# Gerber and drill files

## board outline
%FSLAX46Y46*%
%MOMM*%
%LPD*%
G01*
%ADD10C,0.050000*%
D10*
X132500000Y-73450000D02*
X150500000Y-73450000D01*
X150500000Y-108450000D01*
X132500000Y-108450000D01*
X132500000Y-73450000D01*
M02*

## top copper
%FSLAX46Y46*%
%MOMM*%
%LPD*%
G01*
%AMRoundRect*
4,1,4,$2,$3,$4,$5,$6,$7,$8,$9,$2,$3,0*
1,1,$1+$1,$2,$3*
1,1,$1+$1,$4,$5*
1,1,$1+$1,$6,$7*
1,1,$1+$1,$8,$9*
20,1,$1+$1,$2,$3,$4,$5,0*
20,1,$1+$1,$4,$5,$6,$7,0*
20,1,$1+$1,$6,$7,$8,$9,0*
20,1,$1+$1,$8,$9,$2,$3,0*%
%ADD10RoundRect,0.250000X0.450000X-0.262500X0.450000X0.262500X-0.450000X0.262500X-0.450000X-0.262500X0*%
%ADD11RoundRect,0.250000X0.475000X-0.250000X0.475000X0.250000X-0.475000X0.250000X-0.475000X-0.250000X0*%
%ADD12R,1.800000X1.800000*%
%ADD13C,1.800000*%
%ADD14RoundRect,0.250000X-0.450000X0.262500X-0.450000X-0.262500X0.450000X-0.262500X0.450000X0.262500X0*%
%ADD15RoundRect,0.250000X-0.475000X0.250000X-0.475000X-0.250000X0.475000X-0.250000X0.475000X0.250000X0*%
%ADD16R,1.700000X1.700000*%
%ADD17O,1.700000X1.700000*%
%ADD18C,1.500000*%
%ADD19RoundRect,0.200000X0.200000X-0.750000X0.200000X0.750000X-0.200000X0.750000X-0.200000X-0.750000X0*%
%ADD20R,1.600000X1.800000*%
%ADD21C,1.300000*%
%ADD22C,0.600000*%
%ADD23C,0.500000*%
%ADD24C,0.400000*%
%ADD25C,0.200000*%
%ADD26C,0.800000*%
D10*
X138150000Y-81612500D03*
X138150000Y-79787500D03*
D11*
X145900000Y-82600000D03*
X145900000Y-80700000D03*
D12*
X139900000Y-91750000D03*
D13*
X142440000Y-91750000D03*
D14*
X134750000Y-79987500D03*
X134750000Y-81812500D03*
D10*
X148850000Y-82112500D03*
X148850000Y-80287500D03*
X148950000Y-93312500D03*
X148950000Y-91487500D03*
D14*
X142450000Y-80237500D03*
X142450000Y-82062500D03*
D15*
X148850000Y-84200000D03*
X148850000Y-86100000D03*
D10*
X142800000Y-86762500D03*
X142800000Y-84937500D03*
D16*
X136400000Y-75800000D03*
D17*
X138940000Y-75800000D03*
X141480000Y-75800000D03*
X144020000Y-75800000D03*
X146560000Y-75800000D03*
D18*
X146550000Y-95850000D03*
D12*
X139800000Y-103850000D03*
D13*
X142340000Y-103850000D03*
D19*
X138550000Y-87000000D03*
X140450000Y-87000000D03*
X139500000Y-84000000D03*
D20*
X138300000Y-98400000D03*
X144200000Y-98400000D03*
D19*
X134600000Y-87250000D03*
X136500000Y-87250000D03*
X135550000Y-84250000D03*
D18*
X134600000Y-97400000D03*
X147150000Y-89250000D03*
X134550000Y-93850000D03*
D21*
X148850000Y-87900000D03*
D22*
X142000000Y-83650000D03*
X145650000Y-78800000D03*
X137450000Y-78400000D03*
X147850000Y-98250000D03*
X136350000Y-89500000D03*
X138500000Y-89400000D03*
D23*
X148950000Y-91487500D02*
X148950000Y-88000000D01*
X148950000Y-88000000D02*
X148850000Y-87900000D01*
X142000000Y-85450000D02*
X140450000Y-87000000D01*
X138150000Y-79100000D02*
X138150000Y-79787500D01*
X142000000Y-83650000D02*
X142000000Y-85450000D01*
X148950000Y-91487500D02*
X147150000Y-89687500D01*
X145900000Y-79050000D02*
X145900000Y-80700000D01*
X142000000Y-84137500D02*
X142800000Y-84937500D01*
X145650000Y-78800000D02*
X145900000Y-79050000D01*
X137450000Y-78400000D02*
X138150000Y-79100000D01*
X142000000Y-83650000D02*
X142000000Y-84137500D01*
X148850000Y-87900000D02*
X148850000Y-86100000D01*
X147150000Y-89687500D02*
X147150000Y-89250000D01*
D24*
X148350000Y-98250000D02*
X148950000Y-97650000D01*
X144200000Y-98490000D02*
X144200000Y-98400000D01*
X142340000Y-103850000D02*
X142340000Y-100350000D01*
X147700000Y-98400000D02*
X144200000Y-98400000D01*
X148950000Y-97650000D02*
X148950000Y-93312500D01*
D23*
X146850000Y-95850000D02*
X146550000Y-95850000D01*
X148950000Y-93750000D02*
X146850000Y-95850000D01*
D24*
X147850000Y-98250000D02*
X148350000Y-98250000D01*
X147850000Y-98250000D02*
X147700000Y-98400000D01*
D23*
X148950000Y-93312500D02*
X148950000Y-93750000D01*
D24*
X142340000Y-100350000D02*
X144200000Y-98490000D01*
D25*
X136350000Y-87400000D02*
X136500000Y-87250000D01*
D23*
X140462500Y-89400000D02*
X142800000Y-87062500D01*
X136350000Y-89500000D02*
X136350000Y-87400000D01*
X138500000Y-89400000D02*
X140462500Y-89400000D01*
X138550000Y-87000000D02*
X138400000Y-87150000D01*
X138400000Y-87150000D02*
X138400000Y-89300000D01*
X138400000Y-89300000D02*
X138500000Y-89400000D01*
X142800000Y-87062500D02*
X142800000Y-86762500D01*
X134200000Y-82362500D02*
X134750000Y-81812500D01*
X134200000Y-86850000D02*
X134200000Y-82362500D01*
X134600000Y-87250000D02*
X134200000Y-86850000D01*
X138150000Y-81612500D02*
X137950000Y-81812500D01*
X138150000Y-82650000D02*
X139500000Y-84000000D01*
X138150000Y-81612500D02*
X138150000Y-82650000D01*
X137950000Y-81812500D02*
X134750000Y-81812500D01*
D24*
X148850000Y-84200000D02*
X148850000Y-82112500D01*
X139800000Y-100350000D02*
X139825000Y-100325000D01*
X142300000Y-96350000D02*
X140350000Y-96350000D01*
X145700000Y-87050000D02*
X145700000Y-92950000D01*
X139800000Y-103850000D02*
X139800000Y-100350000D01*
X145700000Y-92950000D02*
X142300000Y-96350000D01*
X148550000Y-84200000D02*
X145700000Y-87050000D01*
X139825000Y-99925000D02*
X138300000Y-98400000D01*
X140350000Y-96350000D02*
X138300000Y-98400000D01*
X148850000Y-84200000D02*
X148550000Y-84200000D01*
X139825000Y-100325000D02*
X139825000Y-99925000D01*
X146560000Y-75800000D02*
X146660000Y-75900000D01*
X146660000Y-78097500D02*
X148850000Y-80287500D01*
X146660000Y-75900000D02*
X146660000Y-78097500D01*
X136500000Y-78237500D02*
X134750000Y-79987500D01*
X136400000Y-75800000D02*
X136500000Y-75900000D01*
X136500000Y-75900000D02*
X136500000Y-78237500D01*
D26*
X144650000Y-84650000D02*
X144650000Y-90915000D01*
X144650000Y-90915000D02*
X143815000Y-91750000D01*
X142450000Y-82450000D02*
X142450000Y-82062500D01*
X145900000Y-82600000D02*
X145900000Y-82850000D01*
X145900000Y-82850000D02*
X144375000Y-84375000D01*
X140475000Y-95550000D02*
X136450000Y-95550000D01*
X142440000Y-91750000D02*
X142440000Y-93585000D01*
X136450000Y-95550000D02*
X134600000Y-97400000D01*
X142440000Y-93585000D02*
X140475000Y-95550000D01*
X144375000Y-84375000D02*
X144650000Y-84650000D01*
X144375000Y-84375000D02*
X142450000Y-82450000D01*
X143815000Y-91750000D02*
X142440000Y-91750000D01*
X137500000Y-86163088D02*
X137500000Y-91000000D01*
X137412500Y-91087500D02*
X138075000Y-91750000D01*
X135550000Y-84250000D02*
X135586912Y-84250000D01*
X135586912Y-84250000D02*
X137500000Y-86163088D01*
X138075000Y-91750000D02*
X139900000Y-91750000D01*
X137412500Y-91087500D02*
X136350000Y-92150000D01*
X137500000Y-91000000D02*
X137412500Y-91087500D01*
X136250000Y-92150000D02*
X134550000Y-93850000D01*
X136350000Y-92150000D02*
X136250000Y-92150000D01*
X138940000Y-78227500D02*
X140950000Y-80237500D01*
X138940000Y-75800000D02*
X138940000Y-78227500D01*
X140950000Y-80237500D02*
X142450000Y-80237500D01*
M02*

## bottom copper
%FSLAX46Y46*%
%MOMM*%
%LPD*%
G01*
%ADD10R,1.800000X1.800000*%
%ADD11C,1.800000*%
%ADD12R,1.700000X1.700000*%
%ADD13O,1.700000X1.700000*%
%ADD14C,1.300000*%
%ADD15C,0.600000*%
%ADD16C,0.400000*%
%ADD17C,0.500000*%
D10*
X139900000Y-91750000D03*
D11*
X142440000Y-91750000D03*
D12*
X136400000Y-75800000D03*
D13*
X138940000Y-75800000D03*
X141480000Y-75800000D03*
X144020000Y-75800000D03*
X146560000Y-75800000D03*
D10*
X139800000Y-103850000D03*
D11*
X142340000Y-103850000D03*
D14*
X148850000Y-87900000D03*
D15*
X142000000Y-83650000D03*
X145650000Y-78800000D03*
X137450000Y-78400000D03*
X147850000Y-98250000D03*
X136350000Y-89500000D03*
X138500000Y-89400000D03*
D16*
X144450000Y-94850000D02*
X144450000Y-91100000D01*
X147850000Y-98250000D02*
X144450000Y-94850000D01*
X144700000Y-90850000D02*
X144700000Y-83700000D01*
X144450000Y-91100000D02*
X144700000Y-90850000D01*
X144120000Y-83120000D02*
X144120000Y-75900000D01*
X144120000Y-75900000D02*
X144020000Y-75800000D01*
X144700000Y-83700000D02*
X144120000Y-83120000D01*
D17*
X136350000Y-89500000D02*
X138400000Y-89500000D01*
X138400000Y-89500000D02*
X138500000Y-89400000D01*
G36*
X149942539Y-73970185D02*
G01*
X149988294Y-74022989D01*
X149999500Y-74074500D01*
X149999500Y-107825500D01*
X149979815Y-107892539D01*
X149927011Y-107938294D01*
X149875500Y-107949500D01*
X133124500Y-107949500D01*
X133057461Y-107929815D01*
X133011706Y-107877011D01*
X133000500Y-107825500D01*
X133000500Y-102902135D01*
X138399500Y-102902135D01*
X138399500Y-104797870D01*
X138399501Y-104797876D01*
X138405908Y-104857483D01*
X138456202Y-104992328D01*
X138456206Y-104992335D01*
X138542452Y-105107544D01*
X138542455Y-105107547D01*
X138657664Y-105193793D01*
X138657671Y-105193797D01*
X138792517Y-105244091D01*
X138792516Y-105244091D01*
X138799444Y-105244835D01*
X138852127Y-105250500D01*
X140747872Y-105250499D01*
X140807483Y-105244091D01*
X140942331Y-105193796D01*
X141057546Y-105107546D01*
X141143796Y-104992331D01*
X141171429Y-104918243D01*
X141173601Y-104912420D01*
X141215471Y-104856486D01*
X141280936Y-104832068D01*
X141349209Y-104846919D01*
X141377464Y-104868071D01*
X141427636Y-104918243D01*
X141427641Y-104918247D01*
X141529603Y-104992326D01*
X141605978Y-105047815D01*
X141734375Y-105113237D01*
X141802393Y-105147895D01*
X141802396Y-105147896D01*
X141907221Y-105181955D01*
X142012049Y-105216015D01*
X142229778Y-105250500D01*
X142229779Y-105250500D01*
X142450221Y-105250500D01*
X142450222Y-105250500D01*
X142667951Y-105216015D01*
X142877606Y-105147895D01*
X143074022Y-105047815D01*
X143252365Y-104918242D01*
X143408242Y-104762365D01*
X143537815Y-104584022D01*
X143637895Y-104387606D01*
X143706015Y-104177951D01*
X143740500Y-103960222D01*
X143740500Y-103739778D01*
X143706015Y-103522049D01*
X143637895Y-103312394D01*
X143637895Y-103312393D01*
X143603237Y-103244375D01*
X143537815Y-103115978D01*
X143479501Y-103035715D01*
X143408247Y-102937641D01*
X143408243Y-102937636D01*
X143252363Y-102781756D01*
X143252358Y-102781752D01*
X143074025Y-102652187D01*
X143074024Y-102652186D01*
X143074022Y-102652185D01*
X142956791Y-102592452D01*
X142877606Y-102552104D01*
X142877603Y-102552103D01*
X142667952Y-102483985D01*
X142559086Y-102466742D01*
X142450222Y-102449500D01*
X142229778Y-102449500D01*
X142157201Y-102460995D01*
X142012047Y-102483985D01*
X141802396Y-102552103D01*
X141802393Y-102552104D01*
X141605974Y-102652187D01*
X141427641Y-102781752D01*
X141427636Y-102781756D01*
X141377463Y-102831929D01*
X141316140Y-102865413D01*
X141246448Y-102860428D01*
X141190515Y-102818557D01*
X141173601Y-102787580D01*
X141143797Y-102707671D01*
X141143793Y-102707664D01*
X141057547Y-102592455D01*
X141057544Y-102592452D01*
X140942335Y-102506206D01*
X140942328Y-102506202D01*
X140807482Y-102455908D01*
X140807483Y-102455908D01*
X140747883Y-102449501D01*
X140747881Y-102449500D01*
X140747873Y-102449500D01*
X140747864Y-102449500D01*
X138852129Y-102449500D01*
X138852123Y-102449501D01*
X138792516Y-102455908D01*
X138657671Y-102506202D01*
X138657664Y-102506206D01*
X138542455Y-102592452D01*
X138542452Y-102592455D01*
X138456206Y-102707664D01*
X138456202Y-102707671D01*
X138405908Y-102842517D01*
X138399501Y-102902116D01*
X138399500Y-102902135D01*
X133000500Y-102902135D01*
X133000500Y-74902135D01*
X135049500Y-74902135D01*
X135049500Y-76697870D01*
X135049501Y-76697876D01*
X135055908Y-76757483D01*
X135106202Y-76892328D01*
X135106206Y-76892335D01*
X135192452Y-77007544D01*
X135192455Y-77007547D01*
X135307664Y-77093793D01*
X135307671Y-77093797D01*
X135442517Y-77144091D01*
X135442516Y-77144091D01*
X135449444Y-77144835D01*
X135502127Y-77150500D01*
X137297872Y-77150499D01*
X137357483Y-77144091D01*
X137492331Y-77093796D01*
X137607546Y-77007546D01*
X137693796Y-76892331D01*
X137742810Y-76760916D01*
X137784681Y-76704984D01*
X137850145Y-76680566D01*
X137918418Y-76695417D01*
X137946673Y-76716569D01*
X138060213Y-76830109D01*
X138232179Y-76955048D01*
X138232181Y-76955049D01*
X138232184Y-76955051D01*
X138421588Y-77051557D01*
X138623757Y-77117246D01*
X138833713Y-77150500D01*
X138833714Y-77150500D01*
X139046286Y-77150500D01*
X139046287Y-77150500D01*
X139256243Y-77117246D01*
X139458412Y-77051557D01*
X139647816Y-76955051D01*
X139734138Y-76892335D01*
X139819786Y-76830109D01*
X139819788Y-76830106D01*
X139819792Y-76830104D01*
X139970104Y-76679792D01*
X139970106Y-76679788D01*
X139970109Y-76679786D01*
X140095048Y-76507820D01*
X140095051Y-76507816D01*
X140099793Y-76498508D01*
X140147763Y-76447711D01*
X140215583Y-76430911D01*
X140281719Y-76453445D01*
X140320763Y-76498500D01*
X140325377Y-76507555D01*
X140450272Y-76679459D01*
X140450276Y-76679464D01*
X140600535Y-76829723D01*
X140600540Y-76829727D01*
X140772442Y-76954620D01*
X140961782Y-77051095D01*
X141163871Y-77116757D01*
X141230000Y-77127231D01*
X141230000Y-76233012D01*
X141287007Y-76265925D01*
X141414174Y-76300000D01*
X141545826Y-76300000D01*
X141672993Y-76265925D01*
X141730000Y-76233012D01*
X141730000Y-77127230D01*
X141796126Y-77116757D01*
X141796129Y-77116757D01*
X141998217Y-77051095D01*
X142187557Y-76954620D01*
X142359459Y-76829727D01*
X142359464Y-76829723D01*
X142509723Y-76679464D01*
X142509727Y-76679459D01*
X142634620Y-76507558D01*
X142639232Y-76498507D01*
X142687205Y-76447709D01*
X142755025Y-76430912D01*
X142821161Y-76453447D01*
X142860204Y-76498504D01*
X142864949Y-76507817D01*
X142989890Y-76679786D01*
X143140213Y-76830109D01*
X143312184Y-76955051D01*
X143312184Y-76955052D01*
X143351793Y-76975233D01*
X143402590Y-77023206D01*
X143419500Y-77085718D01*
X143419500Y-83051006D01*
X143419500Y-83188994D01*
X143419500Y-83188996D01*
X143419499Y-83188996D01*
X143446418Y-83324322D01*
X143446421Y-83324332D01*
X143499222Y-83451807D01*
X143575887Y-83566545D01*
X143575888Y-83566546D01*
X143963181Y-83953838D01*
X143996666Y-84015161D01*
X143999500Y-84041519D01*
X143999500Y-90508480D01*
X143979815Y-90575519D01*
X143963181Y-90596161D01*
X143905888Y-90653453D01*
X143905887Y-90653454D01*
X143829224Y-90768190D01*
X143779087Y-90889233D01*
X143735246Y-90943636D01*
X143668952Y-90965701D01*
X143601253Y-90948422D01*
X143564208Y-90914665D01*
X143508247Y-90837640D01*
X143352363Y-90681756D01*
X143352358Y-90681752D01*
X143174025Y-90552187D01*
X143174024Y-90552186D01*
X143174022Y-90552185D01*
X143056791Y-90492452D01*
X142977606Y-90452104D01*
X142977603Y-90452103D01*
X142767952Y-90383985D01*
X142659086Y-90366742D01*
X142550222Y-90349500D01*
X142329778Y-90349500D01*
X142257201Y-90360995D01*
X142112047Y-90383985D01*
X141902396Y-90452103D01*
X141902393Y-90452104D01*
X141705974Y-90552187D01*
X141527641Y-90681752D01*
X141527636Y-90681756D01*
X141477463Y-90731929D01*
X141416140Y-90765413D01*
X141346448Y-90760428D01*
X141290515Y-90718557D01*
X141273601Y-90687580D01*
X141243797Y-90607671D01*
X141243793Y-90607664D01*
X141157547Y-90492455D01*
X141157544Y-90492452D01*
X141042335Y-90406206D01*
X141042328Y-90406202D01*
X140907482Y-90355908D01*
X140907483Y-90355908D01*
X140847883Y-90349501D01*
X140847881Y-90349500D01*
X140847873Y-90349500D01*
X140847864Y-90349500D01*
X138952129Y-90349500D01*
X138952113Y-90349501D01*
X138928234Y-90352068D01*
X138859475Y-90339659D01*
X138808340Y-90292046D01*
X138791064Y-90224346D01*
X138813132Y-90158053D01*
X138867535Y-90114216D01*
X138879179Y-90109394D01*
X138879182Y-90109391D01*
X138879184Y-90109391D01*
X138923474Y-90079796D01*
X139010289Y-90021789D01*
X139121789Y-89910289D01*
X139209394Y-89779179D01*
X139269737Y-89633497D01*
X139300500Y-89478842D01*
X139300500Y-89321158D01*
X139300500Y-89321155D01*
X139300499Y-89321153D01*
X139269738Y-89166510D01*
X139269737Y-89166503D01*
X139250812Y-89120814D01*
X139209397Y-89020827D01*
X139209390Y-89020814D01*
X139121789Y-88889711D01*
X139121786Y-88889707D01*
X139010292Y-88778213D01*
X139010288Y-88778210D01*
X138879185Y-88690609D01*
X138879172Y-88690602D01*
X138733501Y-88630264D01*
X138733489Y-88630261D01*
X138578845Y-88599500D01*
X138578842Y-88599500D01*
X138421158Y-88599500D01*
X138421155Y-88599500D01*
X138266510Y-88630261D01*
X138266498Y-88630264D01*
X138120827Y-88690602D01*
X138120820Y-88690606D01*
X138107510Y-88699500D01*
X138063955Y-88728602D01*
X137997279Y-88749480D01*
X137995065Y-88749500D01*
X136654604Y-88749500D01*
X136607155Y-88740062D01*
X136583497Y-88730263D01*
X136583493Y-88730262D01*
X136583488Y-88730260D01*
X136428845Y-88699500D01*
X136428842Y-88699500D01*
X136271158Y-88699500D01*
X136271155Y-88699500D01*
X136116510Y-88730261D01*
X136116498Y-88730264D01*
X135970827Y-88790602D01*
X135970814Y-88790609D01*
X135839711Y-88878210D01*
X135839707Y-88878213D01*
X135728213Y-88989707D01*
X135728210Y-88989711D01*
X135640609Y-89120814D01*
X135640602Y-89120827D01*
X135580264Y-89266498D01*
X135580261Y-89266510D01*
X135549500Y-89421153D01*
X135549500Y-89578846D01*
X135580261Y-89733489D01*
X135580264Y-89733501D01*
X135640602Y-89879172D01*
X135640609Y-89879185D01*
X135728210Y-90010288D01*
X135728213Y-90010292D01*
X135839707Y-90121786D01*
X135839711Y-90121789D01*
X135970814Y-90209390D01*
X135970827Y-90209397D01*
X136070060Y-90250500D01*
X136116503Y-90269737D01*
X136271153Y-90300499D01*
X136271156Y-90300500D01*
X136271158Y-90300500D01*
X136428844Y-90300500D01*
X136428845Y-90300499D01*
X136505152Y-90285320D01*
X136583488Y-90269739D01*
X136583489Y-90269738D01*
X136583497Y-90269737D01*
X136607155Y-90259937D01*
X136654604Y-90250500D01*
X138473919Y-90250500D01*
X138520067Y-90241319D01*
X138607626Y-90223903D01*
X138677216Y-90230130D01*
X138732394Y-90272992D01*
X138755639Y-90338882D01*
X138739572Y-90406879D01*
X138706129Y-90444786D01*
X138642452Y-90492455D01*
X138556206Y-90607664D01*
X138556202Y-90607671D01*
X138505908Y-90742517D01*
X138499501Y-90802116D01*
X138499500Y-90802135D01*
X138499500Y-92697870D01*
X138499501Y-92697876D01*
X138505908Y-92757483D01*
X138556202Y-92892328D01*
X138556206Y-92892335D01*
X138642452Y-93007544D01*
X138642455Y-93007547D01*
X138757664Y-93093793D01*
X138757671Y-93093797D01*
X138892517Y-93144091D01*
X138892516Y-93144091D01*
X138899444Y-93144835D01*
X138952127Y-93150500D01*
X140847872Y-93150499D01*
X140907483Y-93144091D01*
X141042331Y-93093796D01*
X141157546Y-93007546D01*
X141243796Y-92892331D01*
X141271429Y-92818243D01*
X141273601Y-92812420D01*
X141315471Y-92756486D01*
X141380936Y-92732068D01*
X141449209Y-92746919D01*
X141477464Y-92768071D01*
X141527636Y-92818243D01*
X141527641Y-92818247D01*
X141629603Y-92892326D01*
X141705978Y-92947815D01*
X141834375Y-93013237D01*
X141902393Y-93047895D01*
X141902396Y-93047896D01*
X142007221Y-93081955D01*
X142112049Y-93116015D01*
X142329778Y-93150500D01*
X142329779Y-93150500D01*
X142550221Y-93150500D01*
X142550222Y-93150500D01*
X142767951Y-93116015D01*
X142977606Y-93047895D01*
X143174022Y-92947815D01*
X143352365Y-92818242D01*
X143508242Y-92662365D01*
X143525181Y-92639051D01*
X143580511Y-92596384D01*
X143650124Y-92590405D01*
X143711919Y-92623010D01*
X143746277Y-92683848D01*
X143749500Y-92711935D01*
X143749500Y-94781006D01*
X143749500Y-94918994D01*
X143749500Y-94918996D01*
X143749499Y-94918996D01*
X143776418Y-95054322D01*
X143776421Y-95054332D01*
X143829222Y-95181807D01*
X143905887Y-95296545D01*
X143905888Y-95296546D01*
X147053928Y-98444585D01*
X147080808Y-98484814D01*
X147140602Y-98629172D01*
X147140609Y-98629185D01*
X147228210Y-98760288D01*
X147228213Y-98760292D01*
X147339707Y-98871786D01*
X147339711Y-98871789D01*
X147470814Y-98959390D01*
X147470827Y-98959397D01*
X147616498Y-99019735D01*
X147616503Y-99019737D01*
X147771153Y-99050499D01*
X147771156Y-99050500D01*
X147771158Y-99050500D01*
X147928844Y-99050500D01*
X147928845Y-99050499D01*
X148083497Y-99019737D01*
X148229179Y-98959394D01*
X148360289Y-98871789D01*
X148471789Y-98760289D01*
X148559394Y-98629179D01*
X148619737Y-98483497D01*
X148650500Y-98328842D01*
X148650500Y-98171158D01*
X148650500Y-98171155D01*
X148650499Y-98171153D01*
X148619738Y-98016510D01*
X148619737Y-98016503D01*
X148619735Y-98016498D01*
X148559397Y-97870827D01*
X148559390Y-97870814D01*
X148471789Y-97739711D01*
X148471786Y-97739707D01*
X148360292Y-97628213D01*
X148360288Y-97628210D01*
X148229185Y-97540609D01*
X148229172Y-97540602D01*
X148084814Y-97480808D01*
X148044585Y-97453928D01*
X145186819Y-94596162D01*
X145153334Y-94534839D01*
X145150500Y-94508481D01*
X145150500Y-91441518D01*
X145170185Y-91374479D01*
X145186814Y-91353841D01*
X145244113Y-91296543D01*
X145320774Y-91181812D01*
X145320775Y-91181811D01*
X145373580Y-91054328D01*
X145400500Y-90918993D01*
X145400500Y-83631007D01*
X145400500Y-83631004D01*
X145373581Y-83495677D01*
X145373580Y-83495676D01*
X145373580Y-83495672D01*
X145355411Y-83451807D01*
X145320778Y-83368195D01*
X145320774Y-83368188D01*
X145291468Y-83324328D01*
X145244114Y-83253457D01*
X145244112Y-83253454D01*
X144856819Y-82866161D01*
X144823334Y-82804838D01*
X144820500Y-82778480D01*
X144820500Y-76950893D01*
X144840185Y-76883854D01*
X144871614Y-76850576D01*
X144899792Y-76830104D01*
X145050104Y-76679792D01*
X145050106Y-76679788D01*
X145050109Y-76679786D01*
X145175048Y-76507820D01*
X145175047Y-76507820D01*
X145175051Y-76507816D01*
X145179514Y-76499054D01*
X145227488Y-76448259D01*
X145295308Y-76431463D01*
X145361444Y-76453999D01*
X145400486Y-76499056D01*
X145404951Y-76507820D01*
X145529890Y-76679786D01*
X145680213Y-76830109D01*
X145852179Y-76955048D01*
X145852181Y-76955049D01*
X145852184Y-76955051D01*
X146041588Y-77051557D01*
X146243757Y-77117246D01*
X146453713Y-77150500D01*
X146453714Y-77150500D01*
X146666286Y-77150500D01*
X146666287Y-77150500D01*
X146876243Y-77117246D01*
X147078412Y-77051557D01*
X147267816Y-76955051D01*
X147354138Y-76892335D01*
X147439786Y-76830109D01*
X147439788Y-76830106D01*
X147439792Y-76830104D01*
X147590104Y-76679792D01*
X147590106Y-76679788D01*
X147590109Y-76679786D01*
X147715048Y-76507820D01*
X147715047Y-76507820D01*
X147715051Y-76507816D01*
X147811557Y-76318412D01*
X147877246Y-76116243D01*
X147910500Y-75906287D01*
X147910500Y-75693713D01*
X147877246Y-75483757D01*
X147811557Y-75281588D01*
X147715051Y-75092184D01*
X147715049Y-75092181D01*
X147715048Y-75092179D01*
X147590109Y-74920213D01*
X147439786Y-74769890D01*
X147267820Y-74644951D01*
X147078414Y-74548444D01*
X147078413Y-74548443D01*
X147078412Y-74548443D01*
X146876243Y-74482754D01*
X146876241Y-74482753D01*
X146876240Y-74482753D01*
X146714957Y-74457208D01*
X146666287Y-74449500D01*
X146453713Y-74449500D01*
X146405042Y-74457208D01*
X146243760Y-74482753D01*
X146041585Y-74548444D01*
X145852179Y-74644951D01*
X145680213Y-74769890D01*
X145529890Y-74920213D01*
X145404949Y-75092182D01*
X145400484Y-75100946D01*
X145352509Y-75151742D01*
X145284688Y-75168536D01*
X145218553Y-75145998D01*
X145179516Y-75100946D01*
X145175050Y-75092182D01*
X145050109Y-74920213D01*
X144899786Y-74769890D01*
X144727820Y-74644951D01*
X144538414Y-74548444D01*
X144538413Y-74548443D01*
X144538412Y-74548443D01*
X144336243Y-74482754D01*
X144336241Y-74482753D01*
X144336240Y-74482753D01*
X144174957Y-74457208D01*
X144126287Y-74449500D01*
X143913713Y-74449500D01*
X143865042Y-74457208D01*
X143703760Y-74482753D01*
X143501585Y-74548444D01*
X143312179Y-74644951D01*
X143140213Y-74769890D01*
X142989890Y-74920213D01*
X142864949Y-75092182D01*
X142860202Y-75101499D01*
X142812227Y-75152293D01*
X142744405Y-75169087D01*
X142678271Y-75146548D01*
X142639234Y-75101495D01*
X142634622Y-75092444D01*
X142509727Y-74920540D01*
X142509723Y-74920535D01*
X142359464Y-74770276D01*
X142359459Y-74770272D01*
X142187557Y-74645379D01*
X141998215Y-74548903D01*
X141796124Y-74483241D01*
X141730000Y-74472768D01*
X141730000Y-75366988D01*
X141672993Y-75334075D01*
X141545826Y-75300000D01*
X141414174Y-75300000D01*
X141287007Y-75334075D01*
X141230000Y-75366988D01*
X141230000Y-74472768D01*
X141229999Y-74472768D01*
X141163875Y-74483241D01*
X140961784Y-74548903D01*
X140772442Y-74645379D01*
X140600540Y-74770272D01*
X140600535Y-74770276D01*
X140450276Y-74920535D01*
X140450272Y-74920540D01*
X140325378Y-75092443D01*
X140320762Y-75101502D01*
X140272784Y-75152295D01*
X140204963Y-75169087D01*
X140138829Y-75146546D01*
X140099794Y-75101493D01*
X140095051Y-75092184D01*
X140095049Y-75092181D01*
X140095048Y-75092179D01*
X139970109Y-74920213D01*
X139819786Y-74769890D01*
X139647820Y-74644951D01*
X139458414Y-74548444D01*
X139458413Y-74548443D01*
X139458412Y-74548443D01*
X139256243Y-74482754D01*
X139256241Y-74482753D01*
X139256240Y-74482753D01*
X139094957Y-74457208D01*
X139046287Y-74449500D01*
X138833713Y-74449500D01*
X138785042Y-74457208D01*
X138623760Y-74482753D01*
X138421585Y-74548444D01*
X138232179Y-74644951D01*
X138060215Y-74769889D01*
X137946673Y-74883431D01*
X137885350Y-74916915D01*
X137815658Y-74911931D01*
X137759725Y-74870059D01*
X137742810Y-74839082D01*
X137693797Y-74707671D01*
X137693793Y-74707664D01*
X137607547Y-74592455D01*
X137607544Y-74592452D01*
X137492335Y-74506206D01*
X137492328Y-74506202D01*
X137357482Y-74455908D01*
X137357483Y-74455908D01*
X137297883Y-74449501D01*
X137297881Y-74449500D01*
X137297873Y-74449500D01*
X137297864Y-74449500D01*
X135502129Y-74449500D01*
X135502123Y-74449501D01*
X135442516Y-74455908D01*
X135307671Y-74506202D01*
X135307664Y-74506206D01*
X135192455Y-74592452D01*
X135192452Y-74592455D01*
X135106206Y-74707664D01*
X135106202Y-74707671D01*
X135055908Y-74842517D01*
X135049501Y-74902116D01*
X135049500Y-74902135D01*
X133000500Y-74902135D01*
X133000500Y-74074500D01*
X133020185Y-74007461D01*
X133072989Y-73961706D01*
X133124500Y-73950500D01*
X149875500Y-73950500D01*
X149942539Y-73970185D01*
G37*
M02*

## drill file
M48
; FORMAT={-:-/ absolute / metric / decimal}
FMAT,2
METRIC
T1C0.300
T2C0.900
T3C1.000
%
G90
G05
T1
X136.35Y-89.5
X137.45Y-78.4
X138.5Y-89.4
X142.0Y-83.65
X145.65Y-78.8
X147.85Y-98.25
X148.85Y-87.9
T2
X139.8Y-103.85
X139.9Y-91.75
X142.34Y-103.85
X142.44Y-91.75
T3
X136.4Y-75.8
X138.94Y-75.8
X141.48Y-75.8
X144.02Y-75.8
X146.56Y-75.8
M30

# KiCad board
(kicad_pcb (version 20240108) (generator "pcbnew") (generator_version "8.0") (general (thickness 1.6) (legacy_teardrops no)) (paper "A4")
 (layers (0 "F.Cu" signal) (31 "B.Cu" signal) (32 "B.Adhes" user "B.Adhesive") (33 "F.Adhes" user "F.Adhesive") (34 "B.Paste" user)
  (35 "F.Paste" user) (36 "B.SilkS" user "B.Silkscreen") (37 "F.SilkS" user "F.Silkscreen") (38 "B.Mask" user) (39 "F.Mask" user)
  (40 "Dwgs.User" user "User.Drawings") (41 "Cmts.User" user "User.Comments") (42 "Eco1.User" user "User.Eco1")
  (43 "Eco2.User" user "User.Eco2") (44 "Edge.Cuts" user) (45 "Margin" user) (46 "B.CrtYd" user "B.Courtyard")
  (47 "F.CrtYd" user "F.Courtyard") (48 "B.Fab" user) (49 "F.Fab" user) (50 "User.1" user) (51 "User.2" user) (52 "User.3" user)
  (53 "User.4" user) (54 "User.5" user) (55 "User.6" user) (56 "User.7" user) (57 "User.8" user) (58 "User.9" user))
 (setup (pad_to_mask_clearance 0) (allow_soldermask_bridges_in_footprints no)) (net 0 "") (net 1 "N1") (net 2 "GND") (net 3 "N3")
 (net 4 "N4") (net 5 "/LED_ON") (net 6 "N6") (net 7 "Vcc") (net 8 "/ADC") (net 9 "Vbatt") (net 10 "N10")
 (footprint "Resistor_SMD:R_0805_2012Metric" (layer "F.Cu") (at 138.15 80.7 90)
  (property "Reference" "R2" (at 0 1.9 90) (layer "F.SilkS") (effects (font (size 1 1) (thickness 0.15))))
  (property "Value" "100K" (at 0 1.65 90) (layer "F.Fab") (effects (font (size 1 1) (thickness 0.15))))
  (pad "1" smd roundrect (at -0.9125 0 90) (size 1.025 1.4) (layers "F.Cu" "F.Paste" "F.Mask") (roundrect_rratio 0.243902) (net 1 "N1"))
  (pad "2" smd roundrect (at 0.9125 0 90) (size 1.025 1.4) (layers "F.Cu" "F.Paste" "F.Mask") (roundrect_rratio 0.243902) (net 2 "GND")))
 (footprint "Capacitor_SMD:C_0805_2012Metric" (layer "F.Cu") (at 145.9 81.65 90)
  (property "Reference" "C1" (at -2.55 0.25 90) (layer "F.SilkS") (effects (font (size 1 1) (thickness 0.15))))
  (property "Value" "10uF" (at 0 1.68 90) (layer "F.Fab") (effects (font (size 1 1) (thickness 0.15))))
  (pad "1" smd roundrect (at -0.95 0 90) (size 1 1.45) (layers "F.Cu" "F.Paste" "F.Mask") (roundrect_rratio 0.25) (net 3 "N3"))
  (pad "2" smd roundrect (at 0.95 0 90) (size 1 1.45) (layers "F.Cu" "F.Paste" "F.Mask") (roundrect_rratio 0.25) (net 2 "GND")))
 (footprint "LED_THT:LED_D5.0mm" (layer "F.Cu") (at 139.9 91.75)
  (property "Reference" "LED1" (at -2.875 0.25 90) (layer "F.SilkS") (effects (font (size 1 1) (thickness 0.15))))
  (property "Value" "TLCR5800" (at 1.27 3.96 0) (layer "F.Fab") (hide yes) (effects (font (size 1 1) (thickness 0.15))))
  (pad "1" thru_hole rect (at 0 0) (size 1.8 1.8) (drill 0.9) (layers "*.Cu" "*.Mask") (remove_unused_layers no) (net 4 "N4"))
  (pad "2" thru_hole circle (at 2.54 0) (size 1.8 1.8) (drill 0.9) (layers "*.Cu" "*.Mask") (remove_unused_layers no) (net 3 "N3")))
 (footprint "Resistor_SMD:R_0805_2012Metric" (layer "F.Cu") (at 134.75 80.9 -90)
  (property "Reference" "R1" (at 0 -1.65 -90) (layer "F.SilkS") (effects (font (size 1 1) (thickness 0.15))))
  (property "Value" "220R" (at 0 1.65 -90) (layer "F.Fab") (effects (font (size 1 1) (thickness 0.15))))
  (pad "1" smd roundrect (at -0.9125 0 270) (size 1.025 1.4) (layers "F.Cu" "F.Paste" "F.Mask") (roundrect_rratio 0.243902)
   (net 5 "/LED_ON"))
  (pad "2" smd roundrect (at 0.9125 0 270) (size 1.025 1.4) (layers "F.Cu" "F.Paste" "F.Mask") (roundrect_rratio 0.243902) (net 1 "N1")))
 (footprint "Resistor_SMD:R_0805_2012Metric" (layer "F.Cu") (at 148.85 81.2 90)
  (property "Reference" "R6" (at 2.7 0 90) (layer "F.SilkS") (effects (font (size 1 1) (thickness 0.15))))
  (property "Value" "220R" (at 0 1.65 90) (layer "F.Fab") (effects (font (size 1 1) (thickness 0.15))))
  (pad "1" smd roundrect (at -0.9125 0 90) (size 1.025 1.4) (layers "F.Cu" "F.Paste" "F.Mask") (roundrect_rratio 0.243902) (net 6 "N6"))
  (pad "2" smd roundrect (at 0.9125 0 90) (size 1.025 1.4) (layers "F.Cu" "F.Paste" "F.Mask") (roundrect_rratio 0.243902) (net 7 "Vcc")))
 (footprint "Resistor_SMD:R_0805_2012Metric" (layer "F.Cu") (at 148.95 92.4 90)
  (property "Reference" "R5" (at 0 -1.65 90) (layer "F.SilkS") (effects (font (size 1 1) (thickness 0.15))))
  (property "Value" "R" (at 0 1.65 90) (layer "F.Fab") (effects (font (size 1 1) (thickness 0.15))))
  (pad "1" smd roundrect (at -0.9125 0 90) (size 1.025 1.4) (layers "F.Cu" "F.Paste" "F.Mask") (roundrect_rratio 0.243902) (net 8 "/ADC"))
  (pad "2" smd roundrect (at 0.9125 0 90) (size 1.025 1.4) (layers "F.Cu" "F.Paste" "F.Mask") (roundrect_rratio 0.243902) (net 2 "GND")))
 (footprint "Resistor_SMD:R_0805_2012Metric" (layer "F.Cu") (at 142.45 81.15 -90)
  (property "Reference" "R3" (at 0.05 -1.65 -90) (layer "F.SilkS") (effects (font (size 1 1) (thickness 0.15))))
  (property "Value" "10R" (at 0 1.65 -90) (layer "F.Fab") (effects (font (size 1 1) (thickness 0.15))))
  (pad "1" smd roundrect (at -0.9125 0 270) (size 1.025 1.4) (layers "F.Cu" "F.Paste" "F.Mask") (roundrect_rratio 0.243902) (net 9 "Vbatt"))
  (pad "2" smd roundrect (at 0.9125 0 270) (size 1.025 1.4) (layers "F.Cu" "F.Paste" "F.Mask") (roundrect_rratio 0.243902) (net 3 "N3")))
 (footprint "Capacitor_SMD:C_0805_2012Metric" (layer "F.Cu") (at 148.85 85.15 -90)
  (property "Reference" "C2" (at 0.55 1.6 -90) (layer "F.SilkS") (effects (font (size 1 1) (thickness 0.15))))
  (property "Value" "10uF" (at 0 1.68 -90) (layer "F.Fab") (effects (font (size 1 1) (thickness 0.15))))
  (pad "1" smd roundrect (at -0.95 0 270) (size 1 1.45) (layers "F.Cu" "F.Paste" "F.Mask") (roundrect_rratio 0.25) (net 6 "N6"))
  (pad "2" smd roundrect (at 0.95 0 270) (size 1 1.45) (layers "F.Cu" "F.Paste" "F.Mask") (roundrect_rratio 0.25) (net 2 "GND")))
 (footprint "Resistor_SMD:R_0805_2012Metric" (layer "F.Cu") (at 142.8 85.85 90)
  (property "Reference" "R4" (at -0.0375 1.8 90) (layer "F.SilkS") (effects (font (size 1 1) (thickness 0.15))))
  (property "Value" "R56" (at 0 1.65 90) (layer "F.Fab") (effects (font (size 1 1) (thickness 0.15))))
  (pad "1" smd roundrect (at -0.9125 0 90) (size 1.025 1.4) (layers "F.Cu" "F.Paste" "F.Mask") (roundrect_rratio 0.243902) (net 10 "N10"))
  (pad "2" smd roundrect (at 0.9125 0 90) (size 1.025 1.4) (layers "F.Cu" "F.Paste" "F.Mask") (roundrect_rratio 0.243902) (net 2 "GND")))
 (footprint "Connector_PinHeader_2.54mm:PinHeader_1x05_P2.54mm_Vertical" (layer "F.Cu") (at 136.4 75.8 90)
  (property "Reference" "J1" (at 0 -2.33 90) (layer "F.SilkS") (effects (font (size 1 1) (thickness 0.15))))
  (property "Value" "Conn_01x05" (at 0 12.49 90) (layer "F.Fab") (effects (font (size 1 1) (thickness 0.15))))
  (pad "1" thru_hole rect (at 0 0 90) (size 1.7 1.7) (drill 1) (layers "*.Cu" "*.Mask") (remove_unused_layers no) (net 5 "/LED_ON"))
  (pad "2" thru_hole oval (at 0 2.54 90) (size 1.7 1.7) (drill 1) (layers "*.Cu" "*.Mask") (remove_unused_layers no) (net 9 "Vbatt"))
  (pad "3" thru_hole oval (at 0 5.08 90) (size 1.7 1.7) (drill 1) (layers "*.Cu" "*.Mask") (remove_unused_layers no) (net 2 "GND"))
  (pad "4" thru_hole oval (at 0 7.62 90) (size 1.7 1.7) (drill 1) (layers "*.Cu" "*.Mask") (remove_unused_layers no) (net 8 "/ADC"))
  (pad "5" thru_hole oval (at 0 10.16 90) (size 1.7 1.7) (drill 1) (layers "*.Cu" "*.Mask") (remove_unused_layers no) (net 7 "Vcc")))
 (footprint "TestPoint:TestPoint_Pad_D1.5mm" (layer "F.Cu") (at 146.55 95.85)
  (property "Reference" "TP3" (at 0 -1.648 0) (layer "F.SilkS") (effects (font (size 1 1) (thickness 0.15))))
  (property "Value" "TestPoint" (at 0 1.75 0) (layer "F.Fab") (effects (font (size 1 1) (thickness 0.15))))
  (pad "1" smd circle (at 0 0) (size 1.5 1.5) (layers "F.Cu" "F.Mask") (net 8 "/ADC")))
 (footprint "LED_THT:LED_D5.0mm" (layer "F.Cu") (at 139.8 103.85)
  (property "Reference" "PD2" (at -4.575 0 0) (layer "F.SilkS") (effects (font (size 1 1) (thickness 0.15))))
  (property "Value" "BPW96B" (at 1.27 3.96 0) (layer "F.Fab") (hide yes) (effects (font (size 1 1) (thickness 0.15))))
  (pad "1" thru_hole rect (at 0 0) (size 1.8 1.8) (drill 0.9) (layers "*.Cu" "*.Mask") (remove_unused_layers no) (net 6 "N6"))
  (pad "2" thru_hole circle (at 2.54 0) (size 1.8 1.8) (drill 0.9) (layers "*.Cu" "*.Mask") (remove_unused_layers no) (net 8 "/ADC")))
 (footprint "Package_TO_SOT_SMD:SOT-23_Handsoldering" (layer "F.Cu") (at 139.5 85.5 90)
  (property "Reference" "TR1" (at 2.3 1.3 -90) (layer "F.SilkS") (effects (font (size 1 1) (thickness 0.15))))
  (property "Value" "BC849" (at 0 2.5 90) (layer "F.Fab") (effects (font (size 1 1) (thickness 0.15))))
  (pad "1" smd roundrect (at -1.5 -0.95 90) (size 1.9 0.8) (layers "F.Cu" "F.Paste" "F.Mask") (roundrect_rratio 0.25) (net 10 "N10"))
  (pad "2" smd roundrect (at -1.5 0.95 90) (size 1.9 0.8) (layers "F.Cu" "F.Paste" "F.Mask") (roundrect_rratio 0.25) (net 2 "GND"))
  (pad "3" smd roundrect (at 1.5 0 90) (size 1.9 0.8) (layers "F.Cu" "F.Paste" "F.Mask") (roundrect_rratio 0.25) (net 1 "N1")))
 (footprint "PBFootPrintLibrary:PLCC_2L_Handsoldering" (layer "F.Cu") (at 141.1 98.4)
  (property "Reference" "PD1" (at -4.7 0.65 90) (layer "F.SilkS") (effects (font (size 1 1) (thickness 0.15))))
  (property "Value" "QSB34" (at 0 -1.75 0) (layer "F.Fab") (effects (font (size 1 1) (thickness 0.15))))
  (pad "1" smd rect (at -2.8 0 180) (size 1.6 1.8) (layers "F.Cu" "F.Paste" "F.Mask") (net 6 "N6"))
  (pad "2" smd rect (at 3.1 0 180) (size 1.6 1.8) (layers "F.Cu" "F.Paste" "F.Mask") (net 8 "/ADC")))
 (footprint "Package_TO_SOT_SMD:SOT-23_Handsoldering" (layer "F.Cu") (at 135.55 85.75 90)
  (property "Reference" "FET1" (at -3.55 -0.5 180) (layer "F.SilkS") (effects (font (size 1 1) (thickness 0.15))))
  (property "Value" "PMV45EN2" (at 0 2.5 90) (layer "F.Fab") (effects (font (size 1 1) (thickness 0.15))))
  (pad "1" smd roundrect (at -1.5 -0.95 90) (size 1.9 0.8) (layers "F.Cu" "F.Paste" "F.Mask") (roundrect_rratio 0.25) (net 1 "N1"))
  (pad "2" smd roundrect (at -1.5 0.95 90) (size 1.9 0.8) (layers "F.Cu" "F.Paste" "F.Mask") (roundrect_rratio 0.25) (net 10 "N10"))
  (pad "3" smd roundrect (at 1.5 0 90) (size 1.9 0.8) (layers "F.Cu" "F.Paste" "F.Mask") (roundrect_rratio 0.25) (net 4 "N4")))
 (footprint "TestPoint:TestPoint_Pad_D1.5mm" (layer "F.Cu") (at 134.6 97.4)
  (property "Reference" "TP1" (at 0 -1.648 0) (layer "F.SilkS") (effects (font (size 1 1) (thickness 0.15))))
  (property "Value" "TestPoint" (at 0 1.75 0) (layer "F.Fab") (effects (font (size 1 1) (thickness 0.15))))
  (pad "1" smd circle (at 0 0) (size 1.5 1.5) (layers "F.Cu" "F.Mask") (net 3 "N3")))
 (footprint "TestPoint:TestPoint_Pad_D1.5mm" (layer "F.Cu") (at 147.15 89.25)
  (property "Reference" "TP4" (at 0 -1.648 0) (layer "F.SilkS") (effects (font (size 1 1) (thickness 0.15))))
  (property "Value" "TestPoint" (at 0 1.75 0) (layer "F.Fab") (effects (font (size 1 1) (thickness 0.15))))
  (pad "1" smd circle (at 0 0) (size 1.5 1.5) (layers "F.Cu" "F.Mask") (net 2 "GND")))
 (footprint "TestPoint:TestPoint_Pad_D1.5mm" (layer "F.Cu") (at 134.55 93.85)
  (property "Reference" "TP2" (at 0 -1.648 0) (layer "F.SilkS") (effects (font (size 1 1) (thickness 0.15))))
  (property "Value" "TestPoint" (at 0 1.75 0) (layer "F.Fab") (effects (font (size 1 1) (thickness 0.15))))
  (pad "1" smd circle (at 0 0) (size 1.5 1.5) (layers "F.Cu" "F.Mask") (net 4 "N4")))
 (gr_rect (start 132.5 73.45) (end 150.5 108.45) (stroke (width 0.05) (type default)) (fill none) (layer "Edge.Cuts"))
 (segment (start 148.95 91.4875) (end 148.95 88) (width 0.5) (layer "F.Cu") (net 2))
 (segment (start 148.95 88) (end 148.85 87.9) (width 0.5) (layer "F.Cu") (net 2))
 (segment (start 142 85.45) (end 140.45 87) (width 0.5) (layer "F.Cu") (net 2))
 (segment (start 138.15 79.1) (end 138.15 79.7875) (width 0.5) (layer "F.Cu") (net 2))
 (segment (start 142 83.65) (end 142 85.45) (width 0.5) (layer "F.Cu") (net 2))
 (segment (start 148.95 91.4875) (end 147.15 89.6875) (width 0.5) (layer "F.Cu") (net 2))
 (segment (start 145.9 79.05) (end 145.9 80.7) (width 0.5) (layer "F.Cu") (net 2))
 (segment (start 142 84.1375) (end 142.8 84.9375) (width 0.5) (layer "F.Cu") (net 2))
 (segment (start 145.65 78.8) (end 145.9 79.05) (width 0.5) (layer "F.Cu") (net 2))
 (segment (start 137.45 78.4) (end 138.15 79.1) (width 0.5) (layer "F.Cu") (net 2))
 (segment (start 142 83.65) (end 142 84.1375) (width 0.5) (layer "F.Cu") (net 2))
 (segment (start 148.85 87.9) (end 148.85 86.1) (width 0.5) (layer "F.Cu") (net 2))
 (segment (start 147.15 89.6875) (end 147.15 89.25) (width 0.5) (layer "F.Cu") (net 2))
 (via (at 148.85 87.9) (size 1.3) (drill 0.3) (layers "F.Cu" "B.Cu") (free yes) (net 2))
 (via (at 142 83.65) (size 0.6) (drill 0.3) (layers "F.Cu" "B.Cu") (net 2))
 (via (at 145.65 78.8) (size 0.6) (drill 0.3) (layers "F.Cu" "B.Cu") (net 2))
 (via (at 137.45 78.4) (size 0.6) (drill 0.3) (layers "F.Cu" "B.Cu") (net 2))
 (segment (start 148.35 98.25) (end 148.95 97.65) (width 0.4) (layer "F.Cu") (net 8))
 (segment (start 144.2 98.49) (end 144.2 98.4) (width 0.4) (layer "F.Cu") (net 8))
 (segment (start 142.34 103.85) (end 142.34 100.35) (width 0.4) (layer "F.Cu") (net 8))
 (segment (start 147.7 98.4) (end 144.2 98.4) (width 0.4) (layer "F.Cu") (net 8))
 (segment (start 148.95 97.65) (end 148.95 93.3125) (width 0.4) (layer "F.Cu") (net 8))
 (segment (start 146.85 95.85) (end 146.55 95.85) (width 0.5) (layer "F.Cu") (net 8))
 (segment (start 148.95 93.75) (end 146.85 95.85) (width 0.5) (layer "F.Cu") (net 8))
 (segment (start 147.85 98.25) (end 148.35 98.25) (width 0.4) (layer "F.Cu") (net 8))
 (segment (start 147.85 98.25) (end 147.7 98.4) (width 0.4) (layer "F.Cu") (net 8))
 (segment (start 148.95 93.3125) (end 148.95 93.75) (width 0.5) (layer "F.Cu") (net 8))
 (segment (start 142.34 100.35) (end 144.2 98.49) (width 0.4) (layer "F.Cu") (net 8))
 (via (at 147.85 98.25) (size 0.6) (drill 0.3) (layers "F.Cu" "B.Cu") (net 8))
 (segment (start 144.45 94.85) (end 144.45 91.1) (width 0.4) (layer "B.Cu") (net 8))
 (segment (start 147.85 98.25) (end 144.45 94.85) (width 0.4) (layer "B.Cu") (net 8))
 (segment (start 144.7 90.85) (end 144.7 83.7) (width 0.4) (layer "B.Cu") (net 8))
 (segment (start 144.45 91.1) (end 144.7 90.85) (width 0.4) (layer "B.Cu") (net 8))
 (segment (start 144.12 83.12) (end 144.12 75.9) (width 0.4) (layer "B.Cu") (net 8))
 (segment (start 144.12 75.9) (end 144.02 75.8) (width 0.4) (layer "B.Cu") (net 8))
 (segment (start 144.7 83.7) (end 144.12 83.12) (width 0.4) (layer "B.Cu") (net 8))
 (segment (start 136.35 87.4) (end 136.5 87.25) (width 0.2) (layer "F.Cu") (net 10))
 (segment (start 140.4625 89.4) (end 142.8 87.0625) (width 0.5) (layer "F.Cu") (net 10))
 (segment (start 136.35 89.5) (end 136.35 87.4) (width 0.5) (layer "F.Cu") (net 10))
 (segment (start 138.5 89.4) (end 140.4625 89.4) (width 0.5) (layer "F.Cu") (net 10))
 (segment (start 138.55 87) (end 138.4 87.15) (width 0.5) (layer "F.Cu") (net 10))
 (segment (start 138.4 87.15) (end 138.4 89.3) (width 0.5) (layer "F.Cu") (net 10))
 (segment (start 138.4 89.3) (end 138.5 89.4) (width 0.5) (layer "F.Cu") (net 10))
 (segment (start 142.8 87.0625) (end 142.8 86.7625) (width 0.5) (layer "F.Cu") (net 10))
 (via (at 136.35 89.5) (size 0.6) (drill 0.3) (layers "F.Cu" "B.Cu") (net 10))
 (via (at 138.5 89.4) (size 0.6) (drill 0.3) (layers "F.Cu" "B.Cu") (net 10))
 (segment (start 136.35 89.5) (end 138.4 89.5) (width 0.5) (layer "B.Cu") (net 10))
 (segment (start 138.4 89.5) (end 138.5 89.4) (width 0.5) (layer "B.Cu") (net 10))
 (segment (start 134.2 82.3625) (end 134.75 81.8125) (width 0.5) (layer "F.Cu") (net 1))
 (segment (start 134.2 86.85) (end 134.2 82.3625) (width 0.5) (layer "F.Cu") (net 1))
 (segment (start 134.6 87.25) (end 134.2 86.85) (width 0.5) (layer "F.Cu") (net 1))
 (segment (start 138.15 81.6125) (end 137.95 81.8125) (width 0.5) (layer "F.Cu") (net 1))
 (segment (start 138.15 82.65) (end 139.5 84) (width 0.5) (layer "F.Cu") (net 1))
 (segment (start 138.15 81.6125) (end 138.15 82.65) (width 0.5) (layer "F.Cu") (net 1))
 (segment (start 137.95 81.8125) (end 134.75 81.8125) (width 0.5) (layer "F.Cu") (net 1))
 (segment (start 148.85 84.2) (end 148.85 82.1125) (width 0.4) (layer "F.Cu") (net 6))
 (segment (start 139.8 100.35) (end 139.825 100.325) (width 0.4) (layer "F.Cu") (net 6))
 (segment (start 142.3 96.35) (end 140.35 96.35) (width 0.4) (layer "F.Cu") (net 6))
 (segment (start 145.7 87.05) (end 145.7 92.95) (width 0.4) (layer "F.Cu") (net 6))
 (segment (start 139.8 103.85) (end 139.8 100.35) (width 0.4) (layer "F.Cu") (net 6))
 (segment (start 145.7 92.95) (end 142.3 96.35) (width 0.4) (layer "F.Cu") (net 6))
 (segment (start 148.55 84.2) (end 145.7 87.05) (width 0.4) (layer "F.Cu") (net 6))
 (segment (start 139.825 99.925) (end 138.3 98.4) (width 0.4) (layer "F.Cu") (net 6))
 (segment (start 140.35 96.35) (end 138.3 98.4) (width 0.4) (layer "F.Cu") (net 6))
 (segment (start 148.85 84.2) (end 148.55 84.2) (width 0.4) (layer "F.Cu") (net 6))
 (segment (start 139.825 100.325) (end 139.825 99.925) (width 0.4) (layer "F.Cu") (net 6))
 (segment (start 146.56 75.8) (end 146.66 75.9) (width 0.4) (layer "F.Cu") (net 7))
 (segment (start 146.66 78.0975) (end 148.85 80.2875) (width 0.4) (layer "F.Cu") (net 7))
 (segment (start 146.66 75.9) (end 146.66 78.0975) (width 0.4) (layer "F.Cu") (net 7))
 (segment (start 136.5 78.2375) (end 134.75 79.9875) (width 0.4) (layer "F.Cu") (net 5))
 (segment (start 136.4 75.8) (end 136.5 75.9) (width 0.4) (layer "F.Cu") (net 5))
 (segment (start 136.5 75.9) (end 136.5 78.2375) (width 0.4) (layer "F.Cu") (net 5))
 (segment (start 144.65 84.65) (end 144.65 90.915) (width 0.8) (layer "F.Cu") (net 3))
 (segment (start 144.65 90.915) (end 143.815 91.75) (width 0.8) (layer "F.Cu") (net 3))
 (segment (start 142.45 82.45) (end 142.45 82.0625) (width 0.8) (layer "F.Cu") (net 3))
 (segment (start 145.9 82.6) (end 145.9 82.85) (width 0.8) (layer "F.Cu") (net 3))
 (segment (start 145.9 82.85) (end 144.375 84.375) (width 0.8) (layer "F.Cu") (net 3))
 (segment (start 140.475 95.55) (end 136.45 95.55) (width 0.8) (layer "F.Cu") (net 3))
 (segment (start 142.44 91.75) (end 142.44 93.585) (width 0.8) (layer "F.Cu") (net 3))
 (segment (start 136.45 95.55) (end 134.6 97.4) (width 0.8) (layer "F.Cu") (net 3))
 (segment (start 142.44 93.585) (end 140.475 95.55) (width 0.8) (layer "F.Cu") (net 3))
 (segment (start 144.375 84.375) (end 144.65 84.65) (width 0.8) (layer "F.Cu") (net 3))
 (segment (start 144.375 84.375) (end 142.45 82.45) (width 0.8) (layer "F.Cu") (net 3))
 (segment (start 143.815 91.75) (end 142.44 91.75) (width 0.8) (layer "F.Cu") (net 3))
 (segment (start 137.5 86.163088) (end 137.5 91) (width 0.8) (layer "F.Cu") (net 4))
 (segment (start 137.4125 91.0875) (end 138.075 91.75) (width 0.8) (layer "F.Cu") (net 4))
 (segment (start 135.55 84.25) (end 135.586912 84.25) (width 0.8) (layer "F.Cu") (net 4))
 (segment (start 135.586912 84.25) (end 137.5 86.163088) (width 0.8) (layer "F.Cu") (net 4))
 (segment (start 138.075 91.75) (end 139.9 91.75) (width 0.8) (layer "F.Cu") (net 4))
 (segment (start 137.4125 91.0875) (end 136.35 92.15) (width 0.8) (layer "F.Cu") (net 4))
 (segment (start 137.5 91) (end 137.4125 91.0875) (width 0.8) (layer "F.Cu") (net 4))
 (segment (start 136.25 92.15) (end 134.55 93.85) (width 0.8) (layer "F.Cu") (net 4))
 (segment (start 136.35 92.15) (end 136.25 92.15) (width 0.8) (layer "F.Cu") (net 4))
 (segment (start 138.94 78.2275) (end 140.95 80.2375) (width 0.8) (layer "F.Cu") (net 9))
 (segment (start 138.94 75.8) (end 138.94 78.2275) (width 0.8) (layer "F.Cu") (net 9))
 (segment (start 140.95 80.2375) (end 142.45 80.2375) (width 0.8) (layer "F.Cu") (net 9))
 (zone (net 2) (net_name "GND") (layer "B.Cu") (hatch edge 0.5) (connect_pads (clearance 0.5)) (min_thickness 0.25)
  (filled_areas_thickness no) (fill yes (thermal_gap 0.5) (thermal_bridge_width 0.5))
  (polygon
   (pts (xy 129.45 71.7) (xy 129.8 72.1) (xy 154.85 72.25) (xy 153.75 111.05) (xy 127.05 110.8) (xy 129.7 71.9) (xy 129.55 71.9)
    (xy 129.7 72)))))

